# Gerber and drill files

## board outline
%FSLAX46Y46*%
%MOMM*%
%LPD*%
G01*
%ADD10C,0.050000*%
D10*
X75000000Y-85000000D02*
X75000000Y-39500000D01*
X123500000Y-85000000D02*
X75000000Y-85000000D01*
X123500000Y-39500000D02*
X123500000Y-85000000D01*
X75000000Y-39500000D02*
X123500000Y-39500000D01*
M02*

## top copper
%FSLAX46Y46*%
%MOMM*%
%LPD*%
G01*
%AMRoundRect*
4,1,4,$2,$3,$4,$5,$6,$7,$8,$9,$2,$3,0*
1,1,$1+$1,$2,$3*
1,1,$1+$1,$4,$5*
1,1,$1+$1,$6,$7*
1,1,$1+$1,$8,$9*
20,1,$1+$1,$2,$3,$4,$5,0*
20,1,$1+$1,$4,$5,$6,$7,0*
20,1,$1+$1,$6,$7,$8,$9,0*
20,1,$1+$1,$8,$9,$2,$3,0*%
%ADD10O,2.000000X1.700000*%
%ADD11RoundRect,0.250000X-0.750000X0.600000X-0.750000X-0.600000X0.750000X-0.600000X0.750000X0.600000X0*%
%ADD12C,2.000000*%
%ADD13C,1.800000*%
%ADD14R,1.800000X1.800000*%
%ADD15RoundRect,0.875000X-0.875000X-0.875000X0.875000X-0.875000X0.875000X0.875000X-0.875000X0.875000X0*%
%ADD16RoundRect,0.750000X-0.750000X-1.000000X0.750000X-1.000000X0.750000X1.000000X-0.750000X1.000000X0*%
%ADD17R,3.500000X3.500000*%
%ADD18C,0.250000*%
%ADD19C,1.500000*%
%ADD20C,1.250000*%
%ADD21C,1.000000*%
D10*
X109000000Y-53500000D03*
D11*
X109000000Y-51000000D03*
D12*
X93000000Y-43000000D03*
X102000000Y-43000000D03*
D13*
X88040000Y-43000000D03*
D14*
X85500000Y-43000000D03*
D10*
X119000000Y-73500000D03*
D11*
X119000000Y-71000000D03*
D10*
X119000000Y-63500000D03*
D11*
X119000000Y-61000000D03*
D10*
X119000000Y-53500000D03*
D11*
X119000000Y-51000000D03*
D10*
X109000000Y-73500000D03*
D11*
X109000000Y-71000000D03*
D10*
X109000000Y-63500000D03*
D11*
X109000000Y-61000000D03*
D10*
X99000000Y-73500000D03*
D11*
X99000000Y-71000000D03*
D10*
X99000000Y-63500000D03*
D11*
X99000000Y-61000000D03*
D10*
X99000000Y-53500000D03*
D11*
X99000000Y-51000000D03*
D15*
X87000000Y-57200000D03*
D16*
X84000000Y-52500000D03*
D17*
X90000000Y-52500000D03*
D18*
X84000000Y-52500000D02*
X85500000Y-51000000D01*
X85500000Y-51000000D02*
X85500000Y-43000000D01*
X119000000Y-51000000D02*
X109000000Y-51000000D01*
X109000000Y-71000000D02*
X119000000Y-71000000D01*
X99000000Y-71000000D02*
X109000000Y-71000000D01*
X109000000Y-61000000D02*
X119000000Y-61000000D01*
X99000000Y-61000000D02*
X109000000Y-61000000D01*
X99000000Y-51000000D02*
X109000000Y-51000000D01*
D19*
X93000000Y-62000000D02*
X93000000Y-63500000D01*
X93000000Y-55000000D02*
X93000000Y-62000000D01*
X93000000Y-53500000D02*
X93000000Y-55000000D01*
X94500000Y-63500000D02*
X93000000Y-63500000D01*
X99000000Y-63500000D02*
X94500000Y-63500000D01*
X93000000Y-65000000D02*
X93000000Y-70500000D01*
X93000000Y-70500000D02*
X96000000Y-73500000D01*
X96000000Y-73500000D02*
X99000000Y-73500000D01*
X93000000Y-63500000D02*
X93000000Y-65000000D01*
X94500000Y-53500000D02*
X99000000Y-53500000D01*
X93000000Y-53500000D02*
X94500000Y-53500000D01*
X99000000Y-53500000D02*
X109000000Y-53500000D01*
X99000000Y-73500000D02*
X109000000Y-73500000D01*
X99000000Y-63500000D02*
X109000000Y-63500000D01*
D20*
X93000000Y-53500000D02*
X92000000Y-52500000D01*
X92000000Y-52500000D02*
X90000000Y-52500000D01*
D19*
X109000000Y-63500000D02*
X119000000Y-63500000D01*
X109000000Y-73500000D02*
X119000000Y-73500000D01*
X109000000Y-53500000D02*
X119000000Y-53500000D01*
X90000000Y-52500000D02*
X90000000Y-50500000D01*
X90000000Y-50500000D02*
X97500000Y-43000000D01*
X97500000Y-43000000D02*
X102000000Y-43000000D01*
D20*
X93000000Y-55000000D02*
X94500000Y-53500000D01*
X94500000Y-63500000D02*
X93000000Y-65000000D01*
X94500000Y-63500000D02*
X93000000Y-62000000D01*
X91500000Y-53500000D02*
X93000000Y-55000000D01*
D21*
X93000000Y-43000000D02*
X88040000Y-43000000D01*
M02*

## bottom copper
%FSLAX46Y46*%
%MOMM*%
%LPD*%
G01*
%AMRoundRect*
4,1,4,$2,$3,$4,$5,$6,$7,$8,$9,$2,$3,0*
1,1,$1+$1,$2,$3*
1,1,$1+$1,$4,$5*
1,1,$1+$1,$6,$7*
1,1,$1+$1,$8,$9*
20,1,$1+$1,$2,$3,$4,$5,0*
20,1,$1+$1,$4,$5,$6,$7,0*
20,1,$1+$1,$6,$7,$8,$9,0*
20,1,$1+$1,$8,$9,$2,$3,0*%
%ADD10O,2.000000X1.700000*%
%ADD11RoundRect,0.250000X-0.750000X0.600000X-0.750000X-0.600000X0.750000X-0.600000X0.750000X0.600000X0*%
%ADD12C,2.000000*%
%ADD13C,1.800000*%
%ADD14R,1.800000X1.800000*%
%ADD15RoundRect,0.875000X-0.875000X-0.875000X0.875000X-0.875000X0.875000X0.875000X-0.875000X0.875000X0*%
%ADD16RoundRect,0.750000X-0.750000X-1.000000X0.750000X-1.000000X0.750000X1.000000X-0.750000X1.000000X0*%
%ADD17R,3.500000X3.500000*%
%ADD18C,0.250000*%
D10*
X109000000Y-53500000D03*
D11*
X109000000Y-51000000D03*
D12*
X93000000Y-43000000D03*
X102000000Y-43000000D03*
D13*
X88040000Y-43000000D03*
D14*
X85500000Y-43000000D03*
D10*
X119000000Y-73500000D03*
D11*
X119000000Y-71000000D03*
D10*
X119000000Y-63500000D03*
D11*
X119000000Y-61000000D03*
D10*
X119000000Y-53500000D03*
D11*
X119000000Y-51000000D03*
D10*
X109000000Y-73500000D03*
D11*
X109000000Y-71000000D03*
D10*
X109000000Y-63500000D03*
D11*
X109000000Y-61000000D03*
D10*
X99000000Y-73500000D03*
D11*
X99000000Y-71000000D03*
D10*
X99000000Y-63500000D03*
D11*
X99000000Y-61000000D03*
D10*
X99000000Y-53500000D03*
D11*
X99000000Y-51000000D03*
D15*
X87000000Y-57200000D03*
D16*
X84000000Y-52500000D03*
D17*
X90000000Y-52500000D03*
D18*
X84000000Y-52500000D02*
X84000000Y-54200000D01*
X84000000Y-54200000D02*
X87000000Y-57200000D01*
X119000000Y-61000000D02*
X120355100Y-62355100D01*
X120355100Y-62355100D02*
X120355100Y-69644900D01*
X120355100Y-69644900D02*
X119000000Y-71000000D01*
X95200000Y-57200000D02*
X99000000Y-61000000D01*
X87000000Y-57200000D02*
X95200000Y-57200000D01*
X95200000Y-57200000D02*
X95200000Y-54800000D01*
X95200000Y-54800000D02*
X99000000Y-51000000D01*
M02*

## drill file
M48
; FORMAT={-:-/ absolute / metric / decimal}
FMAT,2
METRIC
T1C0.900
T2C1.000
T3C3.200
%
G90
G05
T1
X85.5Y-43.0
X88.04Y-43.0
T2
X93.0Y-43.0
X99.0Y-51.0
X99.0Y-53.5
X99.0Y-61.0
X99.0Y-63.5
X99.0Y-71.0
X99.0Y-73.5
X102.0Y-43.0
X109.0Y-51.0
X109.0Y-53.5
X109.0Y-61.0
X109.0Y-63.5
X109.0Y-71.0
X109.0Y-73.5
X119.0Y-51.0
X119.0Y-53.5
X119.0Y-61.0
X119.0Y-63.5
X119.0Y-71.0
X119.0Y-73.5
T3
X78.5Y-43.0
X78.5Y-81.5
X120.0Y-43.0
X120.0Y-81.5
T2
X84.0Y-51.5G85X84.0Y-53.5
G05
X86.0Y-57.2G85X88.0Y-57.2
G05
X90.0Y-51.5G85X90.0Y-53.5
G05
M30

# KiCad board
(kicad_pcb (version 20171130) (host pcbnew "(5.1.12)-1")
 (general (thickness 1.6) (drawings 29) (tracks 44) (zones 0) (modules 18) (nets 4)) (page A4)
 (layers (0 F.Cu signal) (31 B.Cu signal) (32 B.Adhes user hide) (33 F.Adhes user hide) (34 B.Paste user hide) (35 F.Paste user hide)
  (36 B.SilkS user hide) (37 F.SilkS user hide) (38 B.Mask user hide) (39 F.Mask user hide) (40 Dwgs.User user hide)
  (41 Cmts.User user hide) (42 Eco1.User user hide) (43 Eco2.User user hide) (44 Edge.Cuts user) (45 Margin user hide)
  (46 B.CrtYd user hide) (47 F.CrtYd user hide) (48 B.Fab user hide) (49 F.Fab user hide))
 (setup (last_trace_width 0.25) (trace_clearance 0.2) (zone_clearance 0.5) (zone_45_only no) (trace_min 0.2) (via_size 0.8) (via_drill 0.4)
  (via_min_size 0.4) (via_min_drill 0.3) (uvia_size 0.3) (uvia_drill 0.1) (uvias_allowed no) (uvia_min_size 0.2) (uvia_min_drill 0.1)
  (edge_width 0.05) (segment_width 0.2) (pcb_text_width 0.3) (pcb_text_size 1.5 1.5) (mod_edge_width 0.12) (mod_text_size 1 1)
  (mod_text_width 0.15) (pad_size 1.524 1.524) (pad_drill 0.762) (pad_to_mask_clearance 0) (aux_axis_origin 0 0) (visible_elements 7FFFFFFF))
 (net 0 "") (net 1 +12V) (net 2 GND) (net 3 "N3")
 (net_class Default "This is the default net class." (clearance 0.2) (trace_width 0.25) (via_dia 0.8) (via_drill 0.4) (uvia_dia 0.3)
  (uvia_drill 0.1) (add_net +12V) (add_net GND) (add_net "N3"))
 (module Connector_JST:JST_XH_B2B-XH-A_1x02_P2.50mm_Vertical (layer F.Cu) (at 109 51 270)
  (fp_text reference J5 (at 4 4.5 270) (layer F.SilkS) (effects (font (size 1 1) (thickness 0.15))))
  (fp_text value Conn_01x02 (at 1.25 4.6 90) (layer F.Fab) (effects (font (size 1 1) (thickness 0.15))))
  (pad 2 thru_hole oval (at 2.5 0 270) (size 1.7 2) (drill 1) (layers *.Cu *.Mask) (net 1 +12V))
  (pad 1 thru_hole roundrect (at 0 0 270) (size 1.7 2) (drill 1) (layers *.Cu *.Mask) (roundrect_rratio 0.1470588235294118) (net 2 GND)))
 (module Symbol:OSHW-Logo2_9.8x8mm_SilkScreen (layer F.Cu) (at 111.5 44)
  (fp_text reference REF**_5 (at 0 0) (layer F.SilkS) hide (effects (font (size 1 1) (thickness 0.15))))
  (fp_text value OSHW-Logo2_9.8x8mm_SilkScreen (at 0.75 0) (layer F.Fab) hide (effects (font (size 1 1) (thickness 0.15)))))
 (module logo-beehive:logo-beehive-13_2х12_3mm (layer F.Cu) (at 88 78)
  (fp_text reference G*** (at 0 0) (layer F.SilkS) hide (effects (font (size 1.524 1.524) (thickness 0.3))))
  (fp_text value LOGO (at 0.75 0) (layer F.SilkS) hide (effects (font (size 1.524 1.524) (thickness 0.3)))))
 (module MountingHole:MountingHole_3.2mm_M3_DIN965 (layer F.Cu) (at 120 81.5)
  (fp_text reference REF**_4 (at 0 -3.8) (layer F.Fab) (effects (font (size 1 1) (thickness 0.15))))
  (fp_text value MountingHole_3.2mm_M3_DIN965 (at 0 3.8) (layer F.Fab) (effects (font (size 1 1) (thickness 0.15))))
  (pad 1 np_thru_hole circle (at 0 0) (size 3.2 3.2) (drill 3.2) (layers *.Cu *.Mask)))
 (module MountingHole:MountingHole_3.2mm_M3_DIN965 (layer F.Cu) (at 78.5 81.5)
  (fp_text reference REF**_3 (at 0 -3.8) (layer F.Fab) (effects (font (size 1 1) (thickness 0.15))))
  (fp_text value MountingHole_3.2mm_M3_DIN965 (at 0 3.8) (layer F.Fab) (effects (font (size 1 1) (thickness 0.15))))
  (pad 1 np_thru_hole circle (at 0 0) (size 3.2 3.2) (drill 3.2) (layers *.Cu *.Mask)))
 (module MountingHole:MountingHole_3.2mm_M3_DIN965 (layer F.Cu) (at 78.5 43)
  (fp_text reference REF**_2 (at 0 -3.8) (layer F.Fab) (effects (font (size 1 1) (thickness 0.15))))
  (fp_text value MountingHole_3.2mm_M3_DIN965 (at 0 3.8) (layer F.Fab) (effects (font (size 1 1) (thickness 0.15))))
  (pad 1 np_thru_hole circle (at 0 0) (size 3.2 3.2) (drill 3.2) (layers *.Cu *.Mask)))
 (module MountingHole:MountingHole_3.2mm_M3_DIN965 (layer F.Cu) (at 120 43)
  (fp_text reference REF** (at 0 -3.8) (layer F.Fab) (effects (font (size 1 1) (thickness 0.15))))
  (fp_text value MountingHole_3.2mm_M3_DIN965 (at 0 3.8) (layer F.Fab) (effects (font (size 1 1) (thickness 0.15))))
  (pad 1 np_thru_hole circle (at 0 0) (size 3.2 3.2) (drill 3.2) (layers *.Cu *.Mask)))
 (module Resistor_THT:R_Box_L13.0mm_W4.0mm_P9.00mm (layer F.Cu) (at 102 43 180)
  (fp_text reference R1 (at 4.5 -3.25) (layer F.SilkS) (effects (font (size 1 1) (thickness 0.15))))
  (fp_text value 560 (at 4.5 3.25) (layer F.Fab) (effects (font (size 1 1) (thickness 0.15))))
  (pad 2 thru_hole circle (at 9 0 180) (size 2 2) (drill 1) (layers *.Cu *.Mask) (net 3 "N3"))
  (pad 1 thru_hole circle (at 0 0 180) (size 2 2) (drill 1) (layers *.Cu *.Mask) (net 1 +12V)))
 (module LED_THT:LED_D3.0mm (layer F.Cu) (at 85.5 43)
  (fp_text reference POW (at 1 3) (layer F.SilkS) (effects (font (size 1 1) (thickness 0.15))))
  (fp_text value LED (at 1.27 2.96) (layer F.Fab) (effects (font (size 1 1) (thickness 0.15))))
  (pad 2 thru_hole circle (at 2.54 0) (size 1.8 1.8) (drill 0.9) (layers *.Cu *.Mask) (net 3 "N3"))
  (pad 1 thru_hole rect (at 0 0) (size 1.8 1.8) (drill 0.9) (layers *.Cu *.Mask) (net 2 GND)))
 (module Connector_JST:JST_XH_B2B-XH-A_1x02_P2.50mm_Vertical (layer F.Cu) (at 119 71 270)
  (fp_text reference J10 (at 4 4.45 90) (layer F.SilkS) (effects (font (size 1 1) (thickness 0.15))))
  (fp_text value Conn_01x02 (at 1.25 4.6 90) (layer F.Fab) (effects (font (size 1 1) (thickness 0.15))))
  (pad 2 thru_hole oval (at 2.5 0 270) (size 1.7 2) (drill 1) (layers *.Cu *.Mask) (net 1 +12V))
  (pad 1 thru_hole roundrect (at 0 0 270) (size 1.7 2) (drill 1) (layers *.Cu *.Mask) (roundrect_rratio 0.1470588235294118) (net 2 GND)))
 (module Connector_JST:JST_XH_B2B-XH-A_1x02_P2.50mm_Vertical (layer F.Cu) (at 119 61 270)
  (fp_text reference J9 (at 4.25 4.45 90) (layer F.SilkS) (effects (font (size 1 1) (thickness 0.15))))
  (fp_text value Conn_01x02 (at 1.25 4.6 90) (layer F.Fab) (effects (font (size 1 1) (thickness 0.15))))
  (pad 2 thru_hole oval (at 2.5 0 270) (size 1.7 2) (drill 1) (layers *.Cu *.Mask) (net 1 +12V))
  (pad 1 thru_hole roundrect (at 0 0 270) (size 1.7 2) (drill 1) (layers *.Cu *.Mask) (roundrect_rratio 0.1470588235294118) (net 2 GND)))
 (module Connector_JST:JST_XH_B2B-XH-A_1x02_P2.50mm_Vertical (layer F.Cu) (at 119 51 270)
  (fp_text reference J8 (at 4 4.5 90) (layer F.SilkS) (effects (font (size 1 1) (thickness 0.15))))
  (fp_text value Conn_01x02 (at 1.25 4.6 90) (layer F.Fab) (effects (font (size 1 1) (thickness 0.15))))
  (pad 2 thru_hole oval (at 2.5 0 270) (size 1.7 2) (drill 1) (layers *.Cu *.Mask) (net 1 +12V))
  (pad 1 thru_hole roundrect (at 0 0 270) (size 1.7 2) (drill 1) (layers *.Cu *.Mask) (roundrect_rratio 0.1470588235294118) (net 2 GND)))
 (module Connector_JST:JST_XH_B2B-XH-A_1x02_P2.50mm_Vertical (layer F.Cu) (at 109 71 270)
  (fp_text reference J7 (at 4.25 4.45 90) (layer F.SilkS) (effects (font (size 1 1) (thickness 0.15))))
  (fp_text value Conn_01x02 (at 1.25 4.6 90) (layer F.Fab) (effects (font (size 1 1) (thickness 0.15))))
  (pad 2 thru_hole oval (at 2.5 0 270) (size 1.7 2) (drill 1) (layers *.Cu *.Mask) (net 1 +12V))
  (pad 1 thru_hole roundrect (at 0 0 270) (size 1.7 2) (drill 1) (layers *.Cu *.Mask) (roundrect_rratio 0.1470588235294118) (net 2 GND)))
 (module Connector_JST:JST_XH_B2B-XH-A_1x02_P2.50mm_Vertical (layer F.Cu) (at 109 61 270)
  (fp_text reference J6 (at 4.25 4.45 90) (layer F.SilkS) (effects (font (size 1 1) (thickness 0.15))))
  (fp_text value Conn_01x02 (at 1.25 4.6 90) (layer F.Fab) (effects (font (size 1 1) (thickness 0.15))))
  (pad 2 thru_hole oval (at 2.5 0 270) (size 1.7 2) (drill 1) (layers *.Cu *.Mask) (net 1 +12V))
  (pad 1 thru_hole roundrect (at 0 0 270) (size 1.7 2) (drill 1) (layers *.Cu *.Mask) (roundrect_rratio 0.1470588235294118) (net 2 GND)))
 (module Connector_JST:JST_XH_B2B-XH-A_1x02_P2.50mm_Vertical (layer F.Cu) (at 99 71 270)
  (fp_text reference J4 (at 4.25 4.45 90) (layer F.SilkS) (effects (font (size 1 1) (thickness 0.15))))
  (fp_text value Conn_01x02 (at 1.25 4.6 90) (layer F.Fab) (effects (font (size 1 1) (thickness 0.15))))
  (pad 2 thru_hole oval (at 2.5 0 270) (size 1.7 2) (drill 1) (layers *.Cu *.Mask) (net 1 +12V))
  (pad 1 thru_hole roundrect (at 0 0 270) (size 1.7 2) (drill 1) (layers *.Cu *.Mask) (roundrect_rratio 0.1470588235294118) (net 2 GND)))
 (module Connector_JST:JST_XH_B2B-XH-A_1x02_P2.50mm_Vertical (layer F.Cu) (at 99 61 270)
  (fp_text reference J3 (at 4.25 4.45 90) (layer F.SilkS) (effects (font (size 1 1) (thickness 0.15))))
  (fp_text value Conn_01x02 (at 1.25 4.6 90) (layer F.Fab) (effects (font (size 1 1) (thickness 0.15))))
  (pad 2 thru_hole oval (at 2.5 0 270) (size 1.7 2) (drill 1) (layers *.Cu *.Mask) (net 1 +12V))
  (pad 1 thru_hole roundrect (at 0 0 270) (size 1.7 2) (drill 1) (layers *.Cu *.Mask) (roundrect_rratio 0.1470588235294118) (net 2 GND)))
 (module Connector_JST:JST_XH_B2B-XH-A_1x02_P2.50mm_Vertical (layer F.Cu) (at 99 51 270)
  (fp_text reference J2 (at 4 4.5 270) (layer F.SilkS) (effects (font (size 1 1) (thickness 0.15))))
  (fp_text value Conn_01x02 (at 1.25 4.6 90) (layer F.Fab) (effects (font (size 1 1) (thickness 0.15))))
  (pad 2 thru_hole oval (at 2.5 0 270) (size 1.7 2) (drill 1) (layers *.Cu *.Mask) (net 1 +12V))
  (pad 1 thru_hole roundrect (at 0 0 270) (size 1.7 2) (drill 1) (layers *.Cu *.Mask) (roundrect_rratio 0.1470588235294118) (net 2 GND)))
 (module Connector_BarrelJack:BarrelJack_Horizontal (layer F.Cu) (at 90 52.5)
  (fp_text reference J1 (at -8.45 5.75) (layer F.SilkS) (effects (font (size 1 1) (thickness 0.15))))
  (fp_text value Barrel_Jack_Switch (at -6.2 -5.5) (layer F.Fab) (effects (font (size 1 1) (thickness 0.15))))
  (pad 3 thru_hole roundrect (at -3 4.7) (size 3.5 3.5) (drill oval 3 1) (layers *.Cu *.Mask) (roundrect_rratio 0.25) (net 2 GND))
  (pad 2 thru_hole roundrect (at -6 0) (size 3 3.5) (drill oval 1 3) (layers *.Cu *.Mask) (roundrect_rratio 0.25) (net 2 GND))
  (pad 1 thru_hole rect (at 0 0) (size 3.5 3.5) (drill oval 1 3) (layers *.Cu *.Mask) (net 1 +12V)))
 (gr_line (start 75 85) (end 75 39.5) (layer Edge.Cuts) (width 0.05))
 (gr_line (start 123.5 85) (end 75 85) (layer Edge.Cuts) (width 0.05))
 (gr_line (start 123.5 39.5) (end 123.5 85) (layer Edge.Cuts) (width 0.05))
 (gr_line (start 75 39.5) (end 123.5 39.5) (layer Edge.Cuts) (width 0.05))
 (segment (start 84 52.5) (end 85.5 51) (width 0.25) (layer F.Cu) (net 2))
 (segment (start 85.5 51) (end 85.5 43) (width 0.25) (layer F.Cu) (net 2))
 (segment (start 84 52.5) (end 84 54.2) (width 0.25) (layer B.Cu) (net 2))
 (segment (start 84 54.2) (end 87 57.2) (width 0.25) (layer B.Cu) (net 2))
 (segment (start 119 61) (end 120.3551 62.3551) (width 0.25) (layer B.Cu) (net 2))
 (segment (start 120.3551 62.3551) (end 120.3551 69.6449) (width 0.25) (layer B.Cu) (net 2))
 (segment (start 120.3551 69.6449) (end 119 71) (width 0.25) (layer B.Cu) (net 2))
 (segment (start 95.2 57.2) (end 99 61) (width 0.25) (layer B.Cu) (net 2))
 (segment (start 87 57.2) (end 95.2 57.2) (width 0.25) (layer B.Cu) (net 2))
 (segment (start 95.2 57.2) (end 95.2 54.8) (width 0.25) (layer B.Cu) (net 2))
 (segment (start 95.2 54.8) (end 99 51) (width 0.25) (layer B.Cu) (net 2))
 (segment (start 119 51) (end 109 51) (width 0.25) (layer F.Cu) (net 2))
 (segment (start 109 71) (end 119 71) (width 0.25) (layer F.Cu) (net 2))
 (segment (start 99 71) (end 109 71) (width 0.25) (layer F.Cu) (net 2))
 (segment (start 109 61) (end 119 61) (width 0.25) (layer F.Cu) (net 2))
 (segment (start 99 61) (end 109 61) (width 0.25) (layer F.Cu) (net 2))
 (segment (start 99 51) (end 109 51) (width 0.25) (layer F.Cu) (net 2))
 (segment (start 93 62) (end 93 63.5) (width 1.5) (layer F.Cu) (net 1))
 (segment (start 93 55) (end 93 62) (width 1.5) (layer F.Cu) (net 1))
 (segment (start 93 53.5) (end 93 55) (width 1.5) (layer F.Cu) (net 1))
 (segment (start 94.5 63.5) (end 93 63.5) (width 1.5) (layer F.Cu) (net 1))
 (segment (start 99 63.5) (end 94.5 63.5) (width 1.5) (layer F.Cu) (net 1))
 (segment (start 93 65) (end 93 70.5) (width 1.5) (layer F.Cu) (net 1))
 (segment (start 93 70.5) (end 96 73.5) (width 1.5) (layer F.Cu) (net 1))
 (segment (start 96 73.5) (end 99 73.5) (width 1.5) (layer F.Cu) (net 1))
 (segment (start 93 63.5) (end 93 65) (width 1.5) (layer F.Cu) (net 1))
 (segment (start 94.5 53.5) (end 99 53.5) (width 1.5) (layer F.Cu) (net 1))
 (segment (start 93 53.5) (end 94.5 53.5) (width 1.5) (layer F.Cu) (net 1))
 (segment (start 99 53.5) (end 109 53.5) (width 1.5) (layer F.Cu) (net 1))
 (segment (start 99 73.5) (end 109 73.5) (width 1.5) (layer F.Cu) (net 1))
 (segment (start 99 63.5) (end 109 63.5) (width 1.5) (layer F.Cu) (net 1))
 (segment (start 93 53.5) (end 92 52.5) (width 1.25) (layer F.Cu) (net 1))
 (segment (start 92 52.5) (end 90 52.5) (width 1.25) (layer F.Cu) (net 1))
 (segment (start 109 63.5) (end 119 63.5) (width 1.5) (layer F.Cu) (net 1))
 (segment (start 109 73.5) (end 119 73.5) (width 1.5) (layer F.Cu) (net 1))
 (segment (start 109 53.5) (end 119 53.5) (width 1.5) (layer F.Cu) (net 1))
 (segment (start 90 52.5) (end 90 50.5) (width 1.5) (layer F.Cu) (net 1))
 (segment (start 90 50.5) (end 97.5 43) (width 1.5) (layer F.Cu) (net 1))
 (segment (start 97.5 43) (end 102 43) (width 1.5) (layer F.Cu) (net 1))
 (segment (start 93 55) (end 94.5 53.5) (width 1.25) (layer F.Cu) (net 1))
 (segment (start 94.5 63.5) (end 93 65) (width 1.25) (layer F.Cu) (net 1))
 (segment (start 94.5 63.5) (end 93 62) (width 1.25) (layer F.Cu) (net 1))
 (segment (start 91.5 53.5) (end 93 55) (width 1.25) (layer F.Cu) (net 1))
 (segment (start 93 43) (end 88.04 43) (width 1) (layer F.Cu) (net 3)))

